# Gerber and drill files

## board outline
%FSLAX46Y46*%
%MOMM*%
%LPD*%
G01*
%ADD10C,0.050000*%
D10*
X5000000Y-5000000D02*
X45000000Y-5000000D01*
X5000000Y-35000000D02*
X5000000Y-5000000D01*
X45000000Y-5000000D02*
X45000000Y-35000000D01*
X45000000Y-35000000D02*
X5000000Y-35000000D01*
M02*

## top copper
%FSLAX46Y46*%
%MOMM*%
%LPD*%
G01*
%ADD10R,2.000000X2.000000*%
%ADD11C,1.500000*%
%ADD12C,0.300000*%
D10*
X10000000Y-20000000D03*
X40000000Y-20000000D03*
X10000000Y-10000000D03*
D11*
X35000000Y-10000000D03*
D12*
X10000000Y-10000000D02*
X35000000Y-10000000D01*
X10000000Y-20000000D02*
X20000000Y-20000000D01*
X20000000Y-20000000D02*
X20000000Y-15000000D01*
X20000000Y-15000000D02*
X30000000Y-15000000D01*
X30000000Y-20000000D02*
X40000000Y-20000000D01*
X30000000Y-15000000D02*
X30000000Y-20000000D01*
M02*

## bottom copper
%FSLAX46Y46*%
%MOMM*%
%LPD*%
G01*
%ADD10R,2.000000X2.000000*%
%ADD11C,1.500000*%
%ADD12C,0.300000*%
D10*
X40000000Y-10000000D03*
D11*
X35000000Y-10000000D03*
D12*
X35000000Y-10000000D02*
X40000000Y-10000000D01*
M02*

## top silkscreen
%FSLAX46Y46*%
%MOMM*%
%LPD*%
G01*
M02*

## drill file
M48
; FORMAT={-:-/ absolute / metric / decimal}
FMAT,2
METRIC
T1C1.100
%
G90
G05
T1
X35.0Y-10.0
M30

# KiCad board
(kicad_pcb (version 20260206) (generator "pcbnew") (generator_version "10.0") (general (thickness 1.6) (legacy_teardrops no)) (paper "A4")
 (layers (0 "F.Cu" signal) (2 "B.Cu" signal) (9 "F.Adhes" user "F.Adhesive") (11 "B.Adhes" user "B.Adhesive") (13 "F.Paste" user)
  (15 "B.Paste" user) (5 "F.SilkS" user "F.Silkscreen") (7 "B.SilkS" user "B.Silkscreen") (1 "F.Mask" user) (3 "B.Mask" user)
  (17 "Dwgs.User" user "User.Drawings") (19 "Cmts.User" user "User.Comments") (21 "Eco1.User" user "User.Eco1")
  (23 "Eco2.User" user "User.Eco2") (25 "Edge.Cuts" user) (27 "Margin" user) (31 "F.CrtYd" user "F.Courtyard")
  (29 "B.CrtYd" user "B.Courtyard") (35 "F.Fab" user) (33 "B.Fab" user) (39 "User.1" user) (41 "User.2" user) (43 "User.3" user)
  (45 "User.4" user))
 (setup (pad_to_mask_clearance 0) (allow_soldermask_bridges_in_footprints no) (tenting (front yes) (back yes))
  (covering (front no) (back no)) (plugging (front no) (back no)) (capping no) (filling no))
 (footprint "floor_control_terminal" (layer "F.Cu") (at 10 20)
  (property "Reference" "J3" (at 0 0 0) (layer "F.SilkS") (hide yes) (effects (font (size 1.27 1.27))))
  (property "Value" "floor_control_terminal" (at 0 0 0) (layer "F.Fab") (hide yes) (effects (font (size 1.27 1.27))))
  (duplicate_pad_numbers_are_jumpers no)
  (pad "1" smd rect (at 0 0) (size 2 2) (layers "F.Cu" "F.Mask" "F.Paste") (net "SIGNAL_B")))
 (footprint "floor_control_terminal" (layer "F.Cu") (at 40 20)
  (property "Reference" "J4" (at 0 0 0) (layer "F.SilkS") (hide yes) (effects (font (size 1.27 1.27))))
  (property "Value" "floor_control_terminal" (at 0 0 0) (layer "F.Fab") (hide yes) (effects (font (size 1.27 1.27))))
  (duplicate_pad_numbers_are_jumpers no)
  (pad "1" smd rect (at 0 0) (size 2 2) (layers "F.Cu" "F.Mask" "F.Paste") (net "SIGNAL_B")))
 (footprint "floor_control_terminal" (layer "F.Cu") (at 10 10)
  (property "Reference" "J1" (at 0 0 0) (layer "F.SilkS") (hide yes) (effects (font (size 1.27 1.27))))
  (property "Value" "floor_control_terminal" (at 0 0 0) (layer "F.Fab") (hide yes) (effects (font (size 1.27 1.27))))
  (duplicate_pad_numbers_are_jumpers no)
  (pad "1" smd rect (at 0 0) (size 2 2) (layers "F.Cu" "F.Mask" "F.Paste") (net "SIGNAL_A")))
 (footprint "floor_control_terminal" (layer "B.Cu") (at 40 10)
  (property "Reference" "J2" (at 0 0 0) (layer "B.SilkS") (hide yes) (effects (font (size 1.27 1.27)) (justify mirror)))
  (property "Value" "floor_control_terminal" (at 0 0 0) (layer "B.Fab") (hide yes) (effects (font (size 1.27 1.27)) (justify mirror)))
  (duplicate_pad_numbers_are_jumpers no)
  (pad "1" smd rect (at 0 0) (size 2 2) (layers "B.Cu" "B.Mask" "B.Paste") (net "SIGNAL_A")))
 (gr_line (start 5 5) (end 45 5) (stroke (width 0.05) (type default)) (layer "Edge.Cuts"))
 (gr_line (start 5 35) (end 5 5) (stroke (width 0.05) (type default)) (layer "Edge.Cuts"))
 (gr_line (start 45 5) (end 45 35) (stroke (width 0.05) (type default)) (layer "Edge.Cuts"))
 (gr_line (start 45 35) (end 5 35) (stroke (width 0.05) (type default)) (layer "Edge.Cuts"))
 (segment (start 10 10) (end 35 10) (width 0.3) (layer "F.Cu") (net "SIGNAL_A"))
 (via (at 35 10) (size 1.5) (drill 1.1) (layers "F.Cu" "B.Cu") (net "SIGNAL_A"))
 (segment (start 35 10) (end 40 10) (width 0.3) (layer "B.Cu") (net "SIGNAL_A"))
 (segment (start 10 20) (end 20 20) (width 0.3) (layer "F.Cu") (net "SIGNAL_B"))
 (segment (start 20 20) (end 20 15) (width 0.3) (layer "F.Cu") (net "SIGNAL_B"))
 (segment (start 20 15) (end 30 15) (width 0.3) (layer "F.Cu") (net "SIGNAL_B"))
 (segment (start 30 20) (end 40 20) (width 0.3) (layer "F.Cu") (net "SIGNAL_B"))
 (segment (start 30 15) (end 30 20) (width 0.3) (layer "F.Cu") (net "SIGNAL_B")))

